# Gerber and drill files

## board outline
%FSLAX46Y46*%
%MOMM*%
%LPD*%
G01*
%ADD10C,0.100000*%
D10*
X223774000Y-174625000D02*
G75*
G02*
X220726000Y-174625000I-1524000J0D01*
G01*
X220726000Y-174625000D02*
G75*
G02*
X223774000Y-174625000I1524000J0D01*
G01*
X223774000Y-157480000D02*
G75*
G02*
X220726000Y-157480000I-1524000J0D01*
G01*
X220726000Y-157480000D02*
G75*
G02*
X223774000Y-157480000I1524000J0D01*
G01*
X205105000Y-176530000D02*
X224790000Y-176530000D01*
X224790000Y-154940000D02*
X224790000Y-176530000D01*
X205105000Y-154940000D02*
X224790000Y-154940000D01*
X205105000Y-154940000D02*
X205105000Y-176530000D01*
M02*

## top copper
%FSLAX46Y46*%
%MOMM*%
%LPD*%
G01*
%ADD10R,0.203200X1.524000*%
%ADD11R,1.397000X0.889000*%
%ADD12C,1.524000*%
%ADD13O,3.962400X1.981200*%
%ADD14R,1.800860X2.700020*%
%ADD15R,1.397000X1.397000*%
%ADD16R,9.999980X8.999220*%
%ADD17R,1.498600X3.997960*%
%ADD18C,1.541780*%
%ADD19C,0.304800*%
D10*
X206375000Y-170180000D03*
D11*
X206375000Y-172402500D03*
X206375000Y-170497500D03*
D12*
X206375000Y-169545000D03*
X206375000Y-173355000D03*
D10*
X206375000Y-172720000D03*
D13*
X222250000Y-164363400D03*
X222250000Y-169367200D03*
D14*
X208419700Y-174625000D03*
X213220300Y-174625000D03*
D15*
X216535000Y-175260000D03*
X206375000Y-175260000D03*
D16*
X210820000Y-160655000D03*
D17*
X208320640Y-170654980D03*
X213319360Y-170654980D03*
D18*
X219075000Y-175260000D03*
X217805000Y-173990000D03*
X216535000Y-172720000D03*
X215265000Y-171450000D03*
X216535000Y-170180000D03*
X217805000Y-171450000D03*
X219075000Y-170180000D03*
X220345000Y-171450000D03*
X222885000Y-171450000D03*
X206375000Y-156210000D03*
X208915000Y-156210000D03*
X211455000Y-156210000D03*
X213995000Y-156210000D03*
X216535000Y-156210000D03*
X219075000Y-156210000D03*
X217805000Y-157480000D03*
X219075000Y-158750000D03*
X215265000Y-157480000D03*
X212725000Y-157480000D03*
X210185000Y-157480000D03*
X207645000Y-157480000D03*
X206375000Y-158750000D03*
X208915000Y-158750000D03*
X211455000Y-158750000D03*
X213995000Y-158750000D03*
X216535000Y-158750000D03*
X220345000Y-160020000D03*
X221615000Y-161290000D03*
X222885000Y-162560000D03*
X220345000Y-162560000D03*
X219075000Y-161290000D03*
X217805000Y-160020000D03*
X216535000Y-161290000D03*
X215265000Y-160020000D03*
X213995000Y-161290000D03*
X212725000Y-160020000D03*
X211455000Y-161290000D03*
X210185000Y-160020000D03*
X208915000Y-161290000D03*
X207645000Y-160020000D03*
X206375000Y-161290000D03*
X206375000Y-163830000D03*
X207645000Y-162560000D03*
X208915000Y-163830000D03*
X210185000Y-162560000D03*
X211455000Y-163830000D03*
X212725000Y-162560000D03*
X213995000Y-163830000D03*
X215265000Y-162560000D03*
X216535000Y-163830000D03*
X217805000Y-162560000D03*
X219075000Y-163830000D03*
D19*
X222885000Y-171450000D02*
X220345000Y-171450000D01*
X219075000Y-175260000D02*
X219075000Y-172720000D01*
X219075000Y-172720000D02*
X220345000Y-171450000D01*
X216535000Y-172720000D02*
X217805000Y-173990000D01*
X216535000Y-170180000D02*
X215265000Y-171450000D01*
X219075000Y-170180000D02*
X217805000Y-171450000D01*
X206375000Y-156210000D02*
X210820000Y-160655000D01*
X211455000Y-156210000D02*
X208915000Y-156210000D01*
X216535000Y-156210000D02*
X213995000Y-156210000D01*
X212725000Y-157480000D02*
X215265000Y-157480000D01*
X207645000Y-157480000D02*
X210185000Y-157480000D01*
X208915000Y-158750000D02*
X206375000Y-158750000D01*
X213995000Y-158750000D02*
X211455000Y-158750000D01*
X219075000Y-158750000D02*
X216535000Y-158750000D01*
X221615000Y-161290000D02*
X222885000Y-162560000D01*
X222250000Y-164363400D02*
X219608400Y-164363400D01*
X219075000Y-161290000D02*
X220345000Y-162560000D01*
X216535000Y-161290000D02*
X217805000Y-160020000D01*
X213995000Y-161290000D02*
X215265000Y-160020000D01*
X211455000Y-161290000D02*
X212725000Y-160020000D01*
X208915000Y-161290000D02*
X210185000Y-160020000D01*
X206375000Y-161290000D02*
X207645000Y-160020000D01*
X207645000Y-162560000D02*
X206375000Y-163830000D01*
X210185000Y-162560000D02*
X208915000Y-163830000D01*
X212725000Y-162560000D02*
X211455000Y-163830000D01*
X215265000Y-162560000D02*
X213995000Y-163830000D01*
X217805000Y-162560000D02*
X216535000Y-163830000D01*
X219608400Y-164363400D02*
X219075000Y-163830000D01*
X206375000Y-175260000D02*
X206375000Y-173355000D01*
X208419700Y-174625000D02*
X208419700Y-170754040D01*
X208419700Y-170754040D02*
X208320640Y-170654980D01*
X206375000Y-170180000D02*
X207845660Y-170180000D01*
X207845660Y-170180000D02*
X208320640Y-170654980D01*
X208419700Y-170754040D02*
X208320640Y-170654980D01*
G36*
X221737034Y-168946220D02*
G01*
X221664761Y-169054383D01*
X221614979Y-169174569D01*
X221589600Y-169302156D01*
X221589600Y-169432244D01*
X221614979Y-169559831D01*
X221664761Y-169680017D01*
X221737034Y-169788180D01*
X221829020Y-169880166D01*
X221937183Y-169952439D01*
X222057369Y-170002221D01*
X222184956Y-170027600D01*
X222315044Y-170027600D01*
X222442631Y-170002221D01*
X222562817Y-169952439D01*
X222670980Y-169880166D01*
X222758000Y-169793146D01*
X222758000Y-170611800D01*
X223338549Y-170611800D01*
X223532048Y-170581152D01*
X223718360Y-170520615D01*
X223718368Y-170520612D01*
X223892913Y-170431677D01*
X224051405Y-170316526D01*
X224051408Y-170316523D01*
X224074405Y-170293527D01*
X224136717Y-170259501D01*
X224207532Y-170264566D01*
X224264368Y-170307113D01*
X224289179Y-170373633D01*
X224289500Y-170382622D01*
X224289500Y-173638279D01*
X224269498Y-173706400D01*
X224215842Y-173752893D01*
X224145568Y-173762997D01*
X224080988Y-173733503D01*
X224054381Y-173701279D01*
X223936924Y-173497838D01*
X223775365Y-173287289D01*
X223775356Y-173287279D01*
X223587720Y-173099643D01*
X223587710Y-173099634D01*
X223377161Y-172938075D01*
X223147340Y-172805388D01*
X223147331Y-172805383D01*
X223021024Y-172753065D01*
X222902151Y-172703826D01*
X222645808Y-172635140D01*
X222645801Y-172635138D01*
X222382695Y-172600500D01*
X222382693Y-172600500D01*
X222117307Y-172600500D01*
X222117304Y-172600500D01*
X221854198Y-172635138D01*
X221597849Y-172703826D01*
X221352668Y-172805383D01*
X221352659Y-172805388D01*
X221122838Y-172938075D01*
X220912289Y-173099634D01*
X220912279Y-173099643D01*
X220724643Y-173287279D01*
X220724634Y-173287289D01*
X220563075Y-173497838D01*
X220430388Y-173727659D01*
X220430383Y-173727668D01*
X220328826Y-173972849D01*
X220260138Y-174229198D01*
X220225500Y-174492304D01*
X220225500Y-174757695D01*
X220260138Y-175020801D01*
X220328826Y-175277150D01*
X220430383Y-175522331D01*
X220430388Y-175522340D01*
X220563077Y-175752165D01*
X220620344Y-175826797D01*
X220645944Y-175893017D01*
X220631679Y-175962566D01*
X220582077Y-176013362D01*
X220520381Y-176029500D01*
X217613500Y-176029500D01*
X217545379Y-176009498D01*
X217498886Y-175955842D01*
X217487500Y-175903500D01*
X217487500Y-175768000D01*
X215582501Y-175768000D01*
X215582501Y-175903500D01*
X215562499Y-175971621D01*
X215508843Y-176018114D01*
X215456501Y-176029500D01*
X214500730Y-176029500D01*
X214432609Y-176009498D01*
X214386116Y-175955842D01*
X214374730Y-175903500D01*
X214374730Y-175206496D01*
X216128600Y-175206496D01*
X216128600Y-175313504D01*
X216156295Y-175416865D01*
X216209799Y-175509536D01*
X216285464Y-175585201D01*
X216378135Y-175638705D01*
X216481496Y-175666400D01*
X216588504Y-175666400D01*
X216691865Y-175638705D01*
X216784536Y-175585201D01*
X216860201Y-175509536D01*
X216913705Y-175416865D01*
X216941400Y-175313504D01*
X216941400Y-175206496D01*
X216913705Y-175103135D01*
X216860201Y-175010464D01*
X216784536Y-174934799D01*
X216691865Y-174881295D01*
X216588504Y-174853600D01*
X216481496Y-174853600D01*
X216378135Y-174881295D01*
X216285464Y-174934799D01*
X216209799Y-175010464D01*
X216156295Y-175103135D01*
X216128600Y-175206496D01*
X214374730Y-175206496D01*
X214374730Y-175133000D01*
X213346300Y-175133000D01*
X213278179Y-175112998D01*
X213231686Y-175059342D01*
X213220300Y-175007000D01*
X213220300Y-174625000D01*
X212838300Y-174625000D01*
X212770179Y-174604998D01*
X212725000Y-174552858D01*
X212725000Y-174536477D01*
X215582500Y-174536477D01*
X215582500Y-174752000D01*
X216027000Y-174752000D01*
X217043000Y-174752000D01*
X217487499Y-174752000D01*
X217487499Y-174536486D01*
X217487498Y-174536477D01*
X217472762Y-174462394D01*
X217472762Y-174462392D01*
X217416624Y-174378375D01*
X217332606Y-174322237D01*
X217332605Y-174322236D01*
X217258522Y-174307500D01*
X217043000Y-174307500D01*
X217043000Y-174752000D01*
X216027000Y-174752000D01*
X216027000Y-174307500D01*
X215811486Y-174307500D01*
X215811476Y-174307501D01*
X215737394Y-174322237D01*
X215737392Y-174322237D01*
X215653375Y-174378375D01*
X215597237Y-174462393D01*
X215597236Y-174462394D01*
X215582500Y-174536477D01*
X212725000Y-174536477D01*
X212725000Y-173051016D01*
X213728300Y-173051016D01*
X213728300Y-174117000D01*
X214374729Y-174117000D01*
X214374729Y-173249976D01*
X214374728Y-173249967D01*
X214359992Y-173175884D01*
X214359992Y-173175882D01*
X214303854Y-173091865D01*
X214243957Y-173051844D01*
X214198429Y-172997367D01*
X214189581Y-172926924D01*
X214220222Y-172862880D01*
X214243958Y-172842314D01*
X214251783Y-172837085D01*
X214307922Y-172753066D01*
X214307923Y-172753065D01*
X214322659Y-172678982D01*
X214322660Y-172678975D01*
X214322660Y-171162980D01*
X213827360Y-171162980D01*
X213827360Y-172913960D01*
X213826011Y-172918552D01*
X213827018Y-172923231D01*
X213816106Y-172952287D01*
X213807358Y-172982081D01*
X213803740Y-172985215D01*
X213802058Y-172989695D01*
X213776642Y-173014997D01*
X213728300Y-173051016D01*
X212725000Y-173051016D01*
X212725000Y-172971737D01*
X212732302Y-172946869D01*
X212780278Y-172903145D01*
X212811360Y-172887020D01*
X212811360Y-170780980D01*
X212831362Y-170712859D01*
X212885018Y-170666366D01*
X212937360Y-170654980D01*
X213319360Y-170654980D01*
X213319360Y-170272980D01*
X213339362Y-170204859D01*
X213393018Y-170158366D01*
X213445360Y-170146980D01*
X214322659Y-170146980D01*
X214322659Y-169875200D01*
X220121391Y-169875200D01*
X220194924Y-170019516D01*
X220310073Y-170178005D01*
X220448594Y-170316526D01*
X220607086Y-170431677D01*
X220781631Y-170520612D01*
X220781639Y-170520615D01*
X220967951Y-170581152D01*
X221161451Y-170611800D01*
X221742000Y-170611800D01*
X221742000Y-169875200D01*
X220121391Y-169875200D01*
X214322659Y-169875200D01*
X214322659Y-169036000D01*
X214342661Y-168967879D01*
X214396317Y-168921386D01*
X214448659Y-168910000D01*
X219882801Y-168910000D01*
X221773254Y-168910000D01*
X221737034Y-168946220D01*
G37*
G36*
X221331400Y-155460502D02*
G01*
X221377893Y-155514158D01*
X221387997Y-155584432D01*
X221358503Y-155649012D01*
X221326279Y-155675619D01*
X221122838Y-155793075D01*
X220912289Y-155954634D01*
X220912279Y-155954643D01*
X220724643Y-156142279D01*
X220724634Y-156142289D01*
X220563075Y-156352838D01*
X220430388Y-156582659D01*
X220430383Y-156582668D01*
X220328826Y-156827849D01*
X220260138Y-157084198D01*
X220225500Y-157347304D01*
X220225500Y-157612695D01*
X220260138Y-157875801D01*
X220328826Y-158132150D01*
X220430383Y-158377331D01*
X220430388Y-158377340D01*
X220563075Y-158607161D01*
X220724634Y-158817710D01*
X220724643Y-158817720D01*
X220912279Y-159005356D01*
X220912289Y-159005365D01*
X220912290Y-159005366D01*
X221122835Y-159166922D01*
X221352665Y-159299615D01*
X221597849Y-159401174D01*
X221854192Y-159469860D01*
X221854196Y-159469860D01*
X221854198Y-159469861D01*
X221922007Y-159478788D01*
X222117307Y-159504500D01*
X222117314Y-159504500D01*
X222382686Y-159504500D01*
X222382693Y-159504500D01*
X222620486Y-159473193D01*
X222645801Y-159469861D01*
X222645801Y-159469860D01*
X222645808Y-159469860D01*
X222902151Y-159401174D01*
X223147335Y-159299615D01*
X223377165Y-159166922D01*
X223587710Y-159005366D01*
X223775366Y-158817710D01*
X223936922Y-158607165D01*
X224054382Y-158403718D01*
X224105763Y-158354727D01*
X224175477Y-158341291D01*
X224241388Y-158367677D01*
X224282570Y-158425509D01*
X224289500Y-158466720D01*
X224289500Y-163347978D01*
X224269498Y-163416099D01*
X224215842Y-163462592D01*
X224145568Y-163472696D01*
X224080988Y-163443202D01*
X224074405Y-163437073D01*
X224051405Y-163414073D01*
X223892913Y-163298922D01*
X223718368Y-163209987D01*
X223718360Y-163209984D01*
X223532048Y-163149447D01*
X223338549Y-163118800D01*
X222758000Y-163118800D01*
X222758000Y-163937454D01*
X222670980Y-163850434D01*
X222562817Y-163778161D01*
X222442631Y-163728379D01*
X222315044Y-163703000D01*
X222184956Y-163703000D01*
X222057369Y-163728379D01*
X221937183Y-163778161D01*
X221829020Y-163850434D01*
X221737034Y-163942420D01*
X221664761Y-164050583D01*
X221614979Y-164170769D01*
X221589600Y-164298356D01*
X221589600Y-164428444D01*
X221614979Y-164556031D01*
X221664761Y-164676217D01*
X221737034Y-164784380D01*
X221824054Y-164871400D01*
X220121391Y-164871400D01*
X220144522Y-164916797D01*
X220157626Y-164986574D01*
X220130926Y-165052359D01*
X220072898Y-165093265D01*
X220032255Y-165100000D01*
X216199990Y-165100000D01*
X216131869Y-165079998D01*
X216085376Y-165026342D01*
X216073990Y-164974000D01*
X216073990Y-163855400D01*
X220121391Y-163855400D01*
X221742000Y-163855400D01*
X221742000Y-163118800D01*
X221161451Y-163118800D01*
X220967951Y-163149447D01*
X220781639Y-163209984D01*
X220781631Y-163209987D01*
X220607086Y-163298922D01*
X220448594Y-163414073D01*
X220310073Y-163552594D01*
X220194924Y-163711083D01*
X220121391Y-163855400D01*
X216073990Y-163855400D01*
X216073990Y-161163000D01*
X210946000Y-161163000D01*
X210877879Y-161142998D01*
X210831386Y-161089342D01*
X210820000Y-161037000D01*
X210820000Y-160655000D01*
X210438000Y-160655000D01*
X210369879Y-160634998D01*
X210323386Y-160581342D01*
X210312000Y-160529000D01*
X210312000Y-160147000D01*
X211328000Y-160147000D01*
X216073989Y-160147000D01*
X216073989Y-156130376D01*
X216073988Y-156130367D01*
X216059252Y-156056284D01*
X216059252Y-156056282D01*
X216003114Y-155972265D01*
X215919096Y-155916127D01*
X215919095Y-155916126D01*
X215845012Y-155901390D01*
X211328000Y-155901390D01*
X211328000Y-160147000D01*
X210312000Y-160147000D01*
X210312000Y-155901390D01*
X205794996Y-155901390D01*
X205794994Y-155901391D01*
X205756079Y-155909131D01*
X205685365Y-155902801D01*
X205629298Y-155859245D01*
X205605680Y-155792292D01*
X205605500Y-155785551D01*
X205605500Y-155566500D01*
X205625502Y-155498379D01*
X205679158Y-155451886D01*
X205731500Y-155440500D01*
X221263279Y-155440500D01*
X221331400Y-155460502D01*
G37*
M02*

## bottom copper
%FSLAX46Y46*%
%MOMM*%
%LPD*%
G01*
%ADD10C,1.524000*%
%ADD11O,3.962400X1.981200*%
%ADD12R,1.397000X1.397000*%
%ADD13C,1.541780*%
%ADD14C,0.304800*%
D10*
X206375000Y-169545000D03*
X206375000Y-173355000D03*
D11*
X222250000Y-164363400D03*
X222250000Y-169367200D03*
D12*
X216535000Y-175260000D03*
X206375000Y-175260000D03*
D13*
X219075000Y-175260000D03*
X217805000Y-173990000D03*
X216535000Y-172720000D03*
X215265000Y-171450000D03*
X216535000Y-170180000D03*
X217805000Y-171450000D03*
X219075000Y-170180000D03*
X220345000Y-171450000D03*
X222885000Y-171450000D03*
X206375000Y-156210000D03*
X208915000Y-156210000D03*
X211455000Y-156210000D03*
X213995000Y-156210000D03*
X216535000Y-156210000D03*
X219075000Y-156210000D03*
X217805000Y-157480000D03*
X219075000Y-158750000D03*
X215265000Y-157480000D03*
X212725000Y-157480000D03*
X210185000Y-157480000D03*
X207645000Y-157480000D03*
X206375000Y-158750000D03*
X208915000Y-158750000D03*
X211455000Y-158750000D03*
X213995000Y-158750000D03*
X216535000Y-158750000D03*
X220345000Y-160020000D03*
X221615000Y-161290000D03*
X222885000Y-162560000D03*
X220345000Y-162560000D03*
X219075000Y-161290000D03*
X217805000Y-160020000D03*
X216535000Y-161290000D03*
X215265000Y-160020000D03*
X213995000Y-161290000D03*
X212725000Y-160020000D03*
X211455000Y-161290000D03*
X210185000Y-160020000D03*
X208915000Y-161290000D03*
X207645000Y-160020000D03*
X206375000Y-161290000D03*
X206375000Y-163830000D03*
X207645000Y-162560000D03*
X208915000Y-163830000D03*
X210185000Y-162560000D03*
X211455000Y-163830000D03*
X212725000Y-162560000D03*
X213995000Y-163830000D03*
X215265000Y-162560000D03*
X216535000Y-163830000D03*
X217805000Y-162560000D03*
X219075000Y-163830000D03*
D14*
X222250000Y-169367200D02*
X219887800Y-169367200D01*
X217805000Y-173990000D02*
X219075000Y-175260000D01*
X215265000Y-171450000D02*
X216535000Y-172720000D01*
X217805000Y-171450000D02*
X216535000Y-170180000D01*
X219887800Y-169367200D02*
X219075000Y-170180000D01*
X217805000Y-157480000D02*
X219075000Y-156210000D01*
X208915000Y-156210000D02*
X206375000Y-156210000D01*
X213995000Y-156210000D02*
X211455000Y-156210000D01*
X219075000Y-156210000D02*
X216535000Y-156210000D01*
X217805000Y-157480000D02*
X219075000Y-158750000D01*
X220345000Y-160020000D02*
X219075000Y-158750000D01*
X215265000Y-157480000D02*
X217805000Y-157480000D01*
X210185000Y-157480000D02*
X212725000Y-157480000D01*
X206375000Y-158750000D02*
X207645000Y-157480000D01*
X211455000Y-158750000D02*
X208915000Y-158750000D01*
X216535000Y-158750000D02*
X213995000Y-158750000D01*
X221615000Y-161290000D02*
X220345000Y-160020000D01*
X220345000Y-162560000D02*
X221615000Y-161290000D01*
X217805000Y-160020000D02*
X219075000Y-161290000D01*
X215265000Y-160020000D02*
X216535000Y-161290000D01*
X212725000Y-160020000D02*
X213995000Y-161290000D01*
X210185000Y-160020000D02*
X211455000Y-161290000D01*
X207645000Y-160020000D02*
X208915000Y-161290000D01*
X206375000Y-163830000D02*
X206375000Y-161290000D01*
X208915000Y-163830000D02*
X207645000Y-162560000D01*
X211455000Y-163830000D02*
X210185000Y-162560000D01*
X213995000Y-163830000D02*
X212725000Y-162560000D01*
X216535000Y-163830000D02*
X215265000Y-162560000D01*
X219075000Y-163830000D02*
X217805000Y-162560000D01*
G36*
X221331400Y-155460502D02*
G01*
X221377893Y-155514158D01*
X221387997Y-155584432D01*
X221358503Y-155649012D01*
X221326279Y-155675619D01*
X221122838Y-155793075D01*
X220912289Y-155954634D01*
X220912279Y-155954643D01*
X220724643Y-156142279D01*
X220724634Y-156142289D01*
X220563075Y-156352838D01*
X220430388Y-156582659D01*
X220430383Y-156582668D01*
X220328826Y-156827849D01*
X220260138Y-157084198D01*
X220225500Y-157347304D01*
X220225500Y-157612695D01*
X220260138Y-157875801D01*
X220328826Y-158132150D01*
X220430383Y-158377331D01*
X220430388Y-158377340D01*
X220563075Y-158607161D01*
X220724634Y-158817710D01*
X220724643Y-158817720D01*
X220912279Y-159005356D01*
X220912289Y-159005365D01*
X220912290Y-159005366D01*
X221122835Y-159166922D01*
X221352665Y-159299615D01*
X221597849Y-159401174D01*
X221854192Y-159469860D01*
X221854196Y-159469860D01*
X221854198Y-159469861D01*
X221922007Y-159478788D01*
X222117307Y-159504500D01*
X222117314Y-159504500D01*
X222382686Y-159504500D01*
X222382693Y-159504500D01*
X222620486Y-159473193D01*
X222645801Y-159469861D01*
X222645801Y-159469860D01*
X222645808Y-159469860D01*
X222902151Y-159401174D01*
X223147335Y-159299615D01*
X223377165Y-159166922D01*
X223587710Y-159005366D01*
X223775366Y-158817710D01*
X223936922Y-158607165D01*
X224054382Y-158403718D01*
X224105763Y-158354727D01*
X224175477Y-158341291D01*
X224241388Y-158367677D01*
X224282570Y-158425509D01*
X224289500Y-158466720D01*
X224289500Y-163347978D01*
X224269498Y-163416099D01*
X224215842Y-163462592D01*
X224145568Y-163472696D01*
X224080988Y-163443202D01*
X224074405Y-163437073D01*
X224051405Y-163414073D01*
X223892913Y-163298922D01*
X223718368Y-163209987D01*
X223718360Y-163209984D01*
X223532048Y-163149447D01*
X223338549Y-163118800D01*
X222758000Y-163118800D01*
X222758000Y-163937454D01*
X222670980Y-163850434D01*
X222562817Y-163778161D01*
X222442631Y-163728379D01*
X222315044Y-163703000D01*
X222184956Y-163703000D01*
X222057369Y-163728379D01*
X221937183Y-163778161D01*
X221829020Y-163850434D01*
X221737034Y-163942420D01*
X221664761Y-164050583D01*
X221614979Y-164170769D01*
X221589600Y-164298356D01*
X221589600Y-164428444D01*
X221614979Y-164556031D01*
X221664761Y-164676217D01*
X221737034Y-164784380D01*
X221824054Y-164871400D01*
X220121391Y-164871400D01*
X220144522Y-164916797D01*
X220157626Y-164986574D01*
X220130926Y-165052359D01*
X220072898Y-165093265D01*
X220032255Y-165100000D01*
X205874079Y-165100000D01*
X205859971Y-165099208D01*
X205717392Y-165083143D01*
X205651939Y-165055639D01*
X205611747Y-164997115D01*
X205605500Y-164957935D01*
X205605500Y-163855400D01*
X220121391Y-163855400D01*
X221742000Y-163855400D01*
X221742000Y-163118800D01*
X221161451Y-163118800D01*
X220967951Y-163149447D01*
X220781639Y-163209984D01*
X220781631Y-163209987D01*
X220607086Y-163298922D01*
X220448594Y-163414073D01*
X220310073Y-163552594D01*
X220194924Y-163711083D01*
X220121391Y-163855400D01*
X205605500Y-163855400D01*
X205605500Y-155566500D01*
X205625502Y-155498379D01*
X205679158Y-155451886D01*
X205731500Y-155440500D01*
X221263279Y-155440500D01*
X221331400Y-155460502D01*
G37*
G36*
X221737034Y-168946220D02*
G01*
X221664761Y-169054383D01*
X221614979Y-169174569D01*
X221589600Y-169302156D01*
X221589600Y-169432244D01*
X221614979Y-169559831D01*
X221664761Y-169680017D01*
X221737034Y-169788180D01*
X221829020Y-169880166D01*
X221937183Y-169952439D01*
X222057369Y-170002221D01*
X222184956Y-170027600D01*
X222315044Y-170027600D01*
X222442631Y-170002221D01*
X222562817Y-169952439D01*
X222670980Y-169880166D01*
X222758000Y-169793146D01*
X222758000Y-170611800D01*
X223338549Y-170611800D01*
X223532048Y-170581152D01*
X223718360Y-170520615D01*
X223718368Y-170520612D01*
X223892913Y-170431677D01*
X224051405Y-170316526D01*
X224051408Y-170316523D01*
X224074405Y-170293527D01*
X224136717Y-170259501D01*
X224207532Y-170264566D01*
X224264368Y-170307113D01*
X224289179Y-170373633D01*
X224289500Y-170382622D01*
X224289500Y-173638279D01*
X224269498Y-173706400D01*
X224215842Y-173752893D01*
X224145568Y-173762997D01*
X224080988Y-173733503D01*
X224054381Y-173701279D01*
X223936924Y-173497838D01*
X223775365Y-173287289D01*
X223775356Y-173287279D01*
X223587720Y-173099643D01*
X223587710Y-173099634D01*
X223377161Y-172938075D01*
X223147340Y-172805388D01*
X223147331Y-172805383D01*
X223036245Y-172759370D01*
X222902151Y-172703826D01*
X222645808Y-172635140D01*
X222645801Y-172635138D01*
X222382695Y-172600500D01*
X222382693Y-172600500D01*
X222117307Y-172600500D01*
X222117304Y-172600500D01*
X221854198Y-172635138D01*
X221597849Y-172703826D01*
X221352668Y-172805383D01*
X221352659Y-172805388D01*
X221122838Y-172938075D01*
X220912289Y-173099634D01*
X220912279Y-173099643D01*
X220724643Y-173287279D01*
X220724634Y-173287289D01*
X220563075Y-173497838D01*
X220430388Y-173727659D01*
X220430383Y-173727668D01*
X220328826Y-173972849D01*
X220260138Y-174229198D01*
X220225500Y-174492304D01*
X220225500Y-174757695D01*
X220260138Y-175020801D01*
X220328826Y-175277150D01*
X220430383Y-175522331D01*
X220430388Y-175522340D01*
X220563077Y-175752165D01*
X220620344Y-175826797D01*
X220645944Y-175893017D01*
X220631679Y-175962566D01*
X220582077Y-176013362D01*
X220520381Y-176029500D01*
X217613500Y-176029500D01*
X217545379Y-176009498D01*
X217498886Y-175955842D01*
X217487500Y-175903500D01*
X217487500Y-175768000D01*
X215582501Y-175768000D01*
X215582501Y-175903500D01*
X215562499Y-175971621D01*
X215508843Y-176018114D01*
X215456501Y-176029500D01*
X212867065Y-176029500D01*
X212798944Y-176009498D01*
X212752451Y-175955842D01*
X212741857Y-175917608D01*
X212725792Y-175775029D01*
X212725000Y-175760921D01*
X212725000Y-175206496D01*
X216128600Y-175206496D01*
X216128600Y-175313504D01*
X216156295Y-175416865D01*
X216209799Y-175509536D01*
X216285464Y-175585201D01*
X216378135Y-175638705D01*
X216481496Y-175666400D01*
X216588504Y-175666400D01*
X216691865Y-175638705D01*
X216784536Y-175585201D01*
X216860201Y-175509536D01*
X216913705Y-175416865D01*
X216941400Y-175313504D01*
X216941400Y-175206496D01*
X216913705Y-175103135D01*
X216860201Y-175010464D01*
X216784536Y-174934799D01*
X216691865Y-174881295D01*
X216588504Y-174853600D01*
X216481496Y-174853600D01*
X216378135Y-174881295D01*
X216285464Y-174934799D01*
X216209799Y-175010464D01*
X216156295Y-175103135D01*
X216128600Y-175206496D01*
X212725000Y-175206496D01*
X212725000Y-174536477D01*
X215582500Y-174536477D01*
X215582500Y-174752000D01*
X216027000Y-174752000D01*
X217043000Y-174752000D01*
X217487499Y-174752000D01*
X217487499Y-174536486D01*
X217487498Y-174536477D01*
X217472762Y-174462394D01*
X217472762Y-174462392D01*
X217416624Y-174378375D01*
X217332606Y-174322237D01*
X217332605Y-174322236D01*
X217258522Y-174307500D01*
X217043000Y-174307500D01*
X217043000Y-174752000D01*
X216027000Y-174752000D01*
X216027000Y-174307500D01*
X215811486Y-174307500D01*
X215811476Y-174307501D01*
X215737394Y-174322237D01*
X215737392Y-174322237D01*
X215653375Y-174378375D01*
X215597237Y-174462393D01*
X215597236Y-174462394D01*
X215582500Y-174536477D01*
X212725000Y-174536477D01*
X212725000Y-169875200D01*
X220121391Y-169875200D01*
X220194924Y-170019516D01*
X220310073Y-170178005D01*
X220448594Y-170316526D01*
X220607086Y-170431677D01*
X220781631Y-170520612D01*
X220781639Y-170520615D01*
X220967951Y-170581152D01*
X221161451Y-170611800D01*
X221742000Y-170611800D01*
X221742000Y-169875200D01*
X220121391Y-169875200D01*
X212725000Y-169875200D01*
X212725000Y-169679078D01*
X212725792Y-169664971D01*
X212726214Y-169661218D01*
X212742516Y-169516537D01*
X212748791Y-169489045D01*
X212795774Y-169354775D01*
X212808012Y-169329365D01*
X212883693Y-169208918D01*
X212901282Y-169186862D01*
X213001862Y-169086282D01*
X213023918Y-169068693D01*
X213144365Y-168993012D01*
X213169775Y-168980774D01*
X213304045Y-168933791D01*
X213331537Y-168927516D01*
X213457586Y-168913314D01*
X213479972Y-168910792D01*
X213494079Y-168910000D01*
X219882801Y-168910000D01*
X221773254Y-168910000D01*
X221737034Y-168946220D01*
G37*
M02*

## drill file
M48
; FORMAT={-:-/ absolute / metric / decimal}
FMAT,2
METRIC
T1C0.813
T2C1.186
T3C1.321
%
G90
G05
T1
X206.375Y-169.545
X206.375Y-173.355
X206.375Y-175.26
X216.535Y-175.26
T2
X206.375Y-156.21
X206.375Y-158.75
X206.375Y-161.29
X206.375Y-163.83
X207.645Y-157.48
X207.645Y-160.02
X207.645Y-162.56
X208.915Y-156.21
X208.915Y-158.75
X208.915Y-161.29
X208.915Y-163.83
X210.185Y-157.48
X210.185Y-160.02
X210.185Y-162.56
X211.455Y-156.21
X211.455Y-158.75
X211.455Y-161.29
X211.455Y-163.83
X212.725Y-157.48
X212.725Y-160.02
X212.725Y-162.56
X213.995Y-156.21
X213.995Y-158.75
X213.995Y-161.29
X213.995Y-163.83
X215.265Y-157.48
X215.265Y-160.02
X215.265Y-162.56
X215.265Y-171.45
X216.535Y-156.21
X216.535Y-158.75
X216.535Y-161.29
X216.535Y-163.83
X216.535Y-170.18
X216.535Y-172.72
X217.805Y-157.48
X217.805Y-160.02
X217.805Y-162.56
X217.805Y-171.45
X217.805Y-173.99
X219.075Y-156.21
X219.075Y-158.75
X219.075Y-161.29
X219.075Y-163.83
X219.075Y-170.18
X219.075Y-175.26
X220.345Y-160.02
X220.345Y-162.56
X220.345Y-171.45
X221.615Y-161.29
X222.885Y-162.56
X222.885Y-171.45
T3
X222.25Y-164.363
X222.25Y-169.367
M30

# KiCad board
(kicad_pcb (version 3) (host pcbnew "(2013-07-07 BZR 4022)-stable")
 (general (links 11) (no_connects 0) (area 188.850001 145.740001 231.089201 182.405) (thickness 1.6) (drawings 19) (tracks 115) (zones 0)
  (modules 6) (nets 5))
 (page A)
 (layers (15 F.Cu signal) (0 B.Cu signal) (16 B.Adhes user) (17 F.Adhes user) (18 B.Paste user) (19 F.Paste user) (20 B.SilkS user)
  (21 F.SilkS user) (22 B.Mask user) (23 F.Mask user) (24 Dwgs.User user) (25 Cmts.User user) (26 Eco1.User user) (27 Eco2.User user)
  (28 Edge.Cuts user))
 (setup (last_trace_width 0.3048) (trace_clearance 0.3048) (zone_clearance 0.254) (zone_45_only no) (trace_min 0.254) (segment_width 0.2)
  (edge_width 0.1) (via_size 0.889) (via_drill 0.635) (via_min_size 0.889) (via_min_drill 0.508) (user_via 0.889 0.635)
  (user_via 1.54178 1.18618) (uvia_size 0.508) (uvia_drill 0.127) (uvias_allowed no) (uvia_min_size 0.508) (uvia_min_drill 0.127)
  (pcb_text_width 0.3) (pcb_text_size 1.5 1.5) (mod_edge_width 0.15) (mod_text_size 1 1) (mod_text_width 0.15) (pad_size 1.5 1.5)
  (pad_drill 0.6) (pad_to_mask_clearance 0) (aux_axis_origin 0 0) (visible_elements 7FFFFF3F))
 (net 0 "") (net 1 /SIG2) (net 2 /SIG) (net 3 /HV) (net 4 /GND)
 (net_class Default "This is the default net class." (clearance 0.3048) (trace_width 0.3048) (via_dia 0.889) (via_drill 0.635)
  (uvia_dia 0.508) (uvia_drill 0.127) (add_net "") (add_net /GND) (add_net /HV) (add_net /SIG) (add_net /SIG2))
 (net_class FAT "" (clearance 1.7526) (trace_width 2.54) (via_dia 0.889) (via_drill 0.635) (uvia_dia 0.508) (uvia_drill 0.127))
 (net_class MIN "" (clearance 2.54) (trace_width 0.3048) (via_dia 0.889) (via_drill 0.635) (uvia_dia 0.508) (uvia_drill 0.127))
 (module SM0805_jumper (layer F.Cu) (at 206.375 171.45 90)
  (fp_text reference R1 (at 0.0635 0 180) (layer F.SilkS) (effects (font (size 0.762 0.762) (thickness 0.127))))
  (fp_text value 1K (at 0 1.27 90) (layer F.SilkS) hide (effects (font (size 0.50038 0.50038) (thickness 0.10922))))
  (pad 2 smd rect (at 1.27 0 90) (size 1.524 0.2032) (layers F.Cu F.Paste F.Mask) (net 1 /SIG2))
  (pad 1 smd rect (at -0.9525 0 90) (size 0.889 1.397) (layers F.Cu F.Paste F.Mask) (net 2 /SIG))
  (pad 2 smd rect (at 0.9525 0 90) (size 0.889 1.397) (layers F.Cu F.Paste F.Mask) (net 1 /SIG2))
  (pad 2 thru_hole circle (at 1.905 0 90) (size 1.524 1.524) (drill 0.8128) (layers *.Cu *.Mask F.SilkS) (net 1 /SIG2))
  (pad 1 thru_hole circle (at -1.905 0 90) (size 1.524 1.524) (drill 0.8128) (layers *.Cu *.Mask F.SilkS) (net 2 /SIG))
  (pad 1 smd rect (at -1.27 0 90) (size 1.524 0.2032) (layers F.Cu F.Paste F.Mask) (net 2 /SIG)))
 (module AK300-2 (layer F.Cu) (at 222.25 166.878 270)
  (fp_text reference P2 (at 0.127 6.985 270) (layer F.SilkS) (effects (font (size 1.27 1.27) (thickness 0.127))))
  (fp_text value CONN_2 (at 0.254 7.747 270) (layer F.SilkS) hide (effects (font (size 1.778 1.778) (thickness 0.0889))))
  (pad 1 thru_hole oval (at -2.5146 0 270) (size 1.9812 3.9624) (drill 1.3208) (layers *.Cu F.Paste F.SilkS F.Mask) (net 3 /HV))
  (pad 2 thru_hole oval (at 2.4892 0 270) (size 1.9812 3.9624) (drill 1.3208) (layers *.Cu F.Paste F.SilkS F.Mask) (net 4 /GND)))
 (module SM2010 (layer F.Cu) (at 210.82 174.625)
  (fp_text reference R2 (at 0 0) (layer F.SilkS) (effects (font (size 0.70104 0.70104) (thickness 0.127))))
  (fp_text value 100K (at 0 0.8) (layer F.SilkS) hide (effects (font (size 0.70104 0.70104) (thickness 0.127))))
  (pad 1 smd rect (at -2.4003 0) (size 1.80086 2.70002) (layers F.Cu F.Paste F.Mask) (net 1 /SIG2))
  (pad 2 smd rect (at 2.4003 0) (size 1.80086 2.70002) (layers F.Cu F.Paste F.Mask) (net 4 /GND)))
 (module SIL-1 (layer F.Cu) (at 216.535 175.26)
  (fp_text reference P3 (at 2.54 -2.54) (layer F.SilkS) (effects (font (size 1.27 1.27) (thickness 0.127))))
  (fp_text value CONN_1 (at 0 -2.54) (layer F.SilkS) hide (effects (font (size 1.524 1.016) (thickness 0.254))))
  (pad 1 thru_hole rect (at 0 0) (size 1.397 1.397) (drill 0.8128) (layers *.Cu *.Mask F.SilkS) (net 4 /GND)))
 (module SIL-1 (layer F.Cu) (at 206.375 175.26 180)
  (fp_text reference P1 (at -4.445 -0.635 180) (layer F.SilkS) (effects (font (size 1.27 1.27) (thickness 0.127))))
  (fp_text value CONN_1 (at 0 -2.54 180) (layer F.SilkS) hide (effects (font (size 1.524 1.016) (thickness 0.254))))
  (pad 1 thru_hole rect (at 0 0 180) (size 1.397 1.397) (drill 0.8128) (layers *.Cu *.Mask F.SilkS) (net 2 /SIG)))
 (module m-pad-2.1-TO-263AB (layer F.Cu) (at 210.82 160.655)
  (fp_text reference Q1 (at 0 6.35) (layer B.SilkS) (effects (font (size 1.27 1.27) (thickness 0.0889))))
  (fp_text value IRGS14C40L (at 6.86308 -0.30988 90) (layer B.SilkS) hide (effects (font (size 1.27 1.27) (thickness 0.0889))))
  (pad 2 smd rect (at 0 0) (size 9.99998 8.99922) (layers F.Cu F.Paste F.Mask) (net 3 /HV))
  (pad 1 smd rect (at -2.49936 9.99998) (size 1.4986 3.99796) (layers F.Cu F.Paste F.Mask) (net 1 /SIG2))
  (pad 3 smd rect (at 2.49936 9.99998) (size 1.4986 3.99796) (layers F.Cu F.Paste F.Mask) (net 4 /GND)))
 (gr_circle (center 222.25 174.625) (end 223.774 174.625) (layer Edge.Cuts) (width 0.1))
 (gr_circle (center 222.25 157.48) (end 223.774 157.48) (layer Edge.Cuts) (width 0.1))
 (gr_line (start 205.105 176.53) (end 224.79 176.53) (angle 90) (layer Edge.Cuts) (width 0.1))
 (gr_line (start 224.79 154.94) (end 224.79 176.53) (angle 90) (layer Edge.Cuts) (width 0.1))
 (gr_line (start 205.105 154.94) (end 224.79 154.94) (angle 90) (layer Edge.Cuts) (width 0.1))
 (gr_line (start 205.105 154.94) (end 205.105 176.53) (angle 90) (layer Edge.Cuts) (width 0.1))
 (segment (start 222.885 171.45) (end 220.345 171.45) (width 0.3048) (layer F.Cu) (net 4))
 (segment (start 219.075 175.26) (end 219.075 172.72) (width 0.3048) (layer F.Cu) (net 4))
 (segment (start 222.25 169.3672) (end 219.8878 169.3672) (width 0.3048) (layer B.Cu) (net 4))
 (segment (start 219.075 172.72) (end 220.345 171.45) (width 0.3048) (layer F.Cu) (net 4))
 (via (at 219.075 175.26) (size 1.54178) (drill 1.18618) (layers F.Cu B.Cu) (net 4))
 (segment (start 217.805 173.99) (end 219.075 175.26) (width 0.3048) (layer B.Cu) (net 4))
 (via (at 217.805 173.99) (size 1.54178) (drill 1.18618) (layers F.Cu B.Cu) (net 4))
 (segment (start 216.535 172.72) (end 217.805 173.99) (width 0.3048) (layer F.Cu) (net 4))
 (via (at 216.535 172.72) (size 1.54178) (drill 1.18618) (layers F.Cu B.Cu) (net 4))
 (segment (start 215.265 171.45) (end 216.535 172.72) (width 0.3048) (layer B.Cu) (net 4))
 (via (at 215.265 171.45) (size 1.54178) (drill 1.18618) (layers F.Cu B.Cu) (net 4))
 (segment (start 216.535 170.18) (end 215.265 171.45) (width 0.3048) (layer F.Cu) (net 4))
 (via (at 216.535 170.18) (size 1.54178) (drill 1.18618) (layers F.Cu B.Cu) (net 4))
 (segment (start 217.805 171.45) (end 216.535 170.18) (width 0.3048) (layer B.Cu) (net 4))
 (via (at 217.805 171.45) (size 1.54178) (drill 1.18618) (layers F.Cu B.Cu) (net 4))
 (segment (start 219.075 170.18) (end 217.805 171.45) (width 0.3048) (layer F.Cu) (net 4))
 (via (at 219.075 170.18) (size 1.54178) (drill 1.18618) (layers F.Cu B.Cu) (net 4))
 (segment (start 219.8878 169.3672) (end 219.075 170.18) (width 0.3048) (layer B.Cu) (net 4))
 (via (at 220.345 171.45) (size 1.54178) (drill 1.18618) (layers F.Cu B.Cu) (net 4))
 (via (at 222.885 171.45) (size 1.54178) (drill 1.18618) (layers F.Cu B.Cu) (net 4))
 (segment (start 217.805 157.48) (end 219.075 156.21) (width 0.3048) (layer B.Cu) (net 3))
 (segment (start 206.375 156.21) (end 210.82 160.655) (width 0.3048) (layer F.Cu) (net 3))
 (via (at 206.375 156.21) (size 1.54178) (drill 1.18618) (layers F.Cu B.Cu) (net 3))
 (segment (start 208.915 156.21) (end 206.375 156.21) (width 0.3048) (layer B.Cu) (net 3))
 (via (at 208.915 156.21) (size 1.54178) (drill 1.18618) (layers F.Cu B.Cu) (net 3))
 (segment (start 211.455 156.21) (end 208.915 156.21) (width 0.3048) (layer F.Cu) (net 3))
 (via (at 211.455 156.21) (size 1.54178) (drill 1.18618) (layers F.Cu B.Cu) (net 3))
 (segment (start 213.995 156.21) (end 211.455 156.21) (width 0.3048) (layer B.Cu) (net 3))
 (via (at 213.995 156.21) (size 1.54178) (drill 1.18618) (layers F.Cu B.Cu) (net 3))
 (segment (start 216.535 156.21) (end 213.995 156.21) (width 0.3048) (layer F.Cu) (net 3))
 (via (at 216.535 156.21) (size 1.54178) (drill 1.18618) (layers F.Cu B.Cu) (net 3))
 (segment (start 219.075 156.21) (end 216.535 156.21) (width 0.3048) (layer B.Cu) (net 3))
 (via (at 219.075 156.21) (size 1.54178) (drill 1.18618) (layers F.Cu B.Cu) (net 3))
 (via (at 217.805 157.48) (size 1.54178) (drill 1.18618) (layers F.Cu B.Cu) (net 3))
 (segment (start 217.805 157.48) (end 219.075 158.75) (width 0.3048) (layer B.Cu) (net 3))
 (segment (start 220.345 160.02) (end 219.075 158.75) (width 0.3048) (layer B.Cu) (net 3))
 (via (at 219.075 158.75) (size 1.54178) (drill 1.18618) (layers F.Cu B.Cu) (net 3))
 (segment (start 215.265 157.48) (end 217.805 157.48) (width 0.3048) (layer B.Cu) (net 3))
 (via (at 215.265 157.48) (size 1.54178) (drill 1.18618) (layers F.Cu B.Cu) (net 3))
 (segment (start 212.725 157.48) (end 215.265 157.48) (width 0.3048) (layer F.Cu) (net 3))
 (via (at 212.725 157.48) (size 1.54178) (drill 1.18618) (layers F.Cu B.Cu) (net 3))
 (segment (start 210.185 157.48) (end 212.725 157.48) (width 0.3048) (layer B.Cu) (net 3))
 (via (at 210.185 157.48) (size 1.54178) (drill 1.18618) (layers F.Cu B.Cu) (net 3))
 (segment (start 207.645 157.48) (end 210.185 157.48) (width 0.3048) (layer F.Cu) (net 3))
 (via (at 207.645 157.48) (size 1.54178) (drill 1.18618) (layers F.Cu B.Cu) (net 3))
 (segment (start 206.375 158.75) (end 207.645 157.48) (width 0.3048) (layer B.Cu) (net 3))
 (via (at 206.375 158.75) (size 1.54178) (drill 1.18618) (layers F.Cu B.Cu) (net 3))
 (segment (start 208.915 158.75) (end 206.375 158.75) (width 0.3048) (layer F.Cu) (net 3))
 (via (at 208.915 158.75) (size 1.54178) (drill 1.18618) (layers F.Cu B.Cu) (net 3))
 (segment (start 211.455 158.75) (end 208.915 158.75) (width 0.3048) (layer B.Cu) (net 3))
 (via (at 211.455 158.75) (size 1.54178) (drill 1.18618) (layers F.Cu B.Cu) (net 3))
 (segment (start 213.995 158.75) (end 211.455 158.75) (width 0.3048) (layer F.Cu) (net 3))
 (via (at 213.995 158.75) (size 1.54178) (drill 1.18618) (layers F.Cu B.Cu) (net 3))
 (segment (start 216.535 158.75) (end 213.995 158.75) (width 0.3048) (layer B.Cu) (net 3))
 (via (at 216.535 158.75) (size 1.54178) (drill 1.18618) (layers F.Cu B.Cu) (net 3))
 (segment (start 219.075 158.75) (end 216.535 158.75) (width 0.3048) (layer F.Cu) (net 3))
 (via (at 220.345 160.02) (size 1.54178) (drill 1.18618) (layers F.Cu B.Cu) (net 3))
 (segment (start 221.615 161.29) (end 220.345 160.02) (width 0.3048) (layer B.Cu) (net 3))
 (via (at 221.615 161.29) (size 1.54178) (drill 1.18618) (layers F.Cu B.Cu) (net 3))
 (via (at 222.885 162.56) (size 1.54178) (drill 1.18618) (layers F.Cu B.Cu) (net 3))
 (segment (start 221.615 161.29) (end 222.885 162.56) (width 0.3048) (layer F.Cu) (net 3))
 (segment (start 222.25 164.3634) (end 219.6084 164.3634) (width 0.3048) (layer F.Cu) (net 3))
 (segment (start 220.345 162.56) (end 221.615 161.29) (width 0.3048) (layer B.Cu) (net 3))
 (via (at 220.345 162.56) (size 1.54178) (drill 1.18618) (layers F.Cu B.Cu) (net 3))
 (segment (start 219.075 161.29) (end 220.345 162.56) (width 0.3048) (layer F.Cu) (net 3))
 (via (at 219.075 161.29) (size 1.54178) (drill 1.18618) (layers F.Cu B.Cu) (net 3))
 (segment (start 217.805 160.02) (end 219.075 161.29) (width 0.3048) (layer B.Cu) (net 3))
 (via (at 217.805 160.02) (size 1.54178) (drill 1.18618) (layers F.Cu B.Cu) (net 3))
 (segment (start 216.535 161.29) (end 217.805 160.02) (width 0.3048) (layer F.Cu) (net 3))
 (via (at 216.535 161.29) (size 1.54178) (drill 1.18618) (layers F.Cu B.Cu) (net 3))
 (segment (start 215.265 160.02) (end 216.535 161.29) (width 0.3048) (layer B.Cu) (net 3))
 (via (at 215.265 160.02) (size 1.54178) (drill 1.18618) (layers F.Cu B.Cu) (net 3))
 (segment (start 213.995 161.29) (end 215.265 160.02) (width 0.3048) (layer F.Cu) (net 3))
 (via (at 213.995 161.29) (size 1.54178) (drill 1.18618) (layers F.Cu B.Cu) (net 3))
 (segment (start 212.725 160.02) (end 213.995 161.29) (width 0.3048) (layer B.Cu) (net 3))
 (via (at 212.725 160.02) (size 1.54178) (drill 1.18618) (layers F.Cu B.Cu) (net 3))
 (segment (start 211.455 161.29) (end 212.725 160.02) (width 0.3048) (layer F.Cu) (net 3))
 (via (at 211.455 161.29) (size 1.54178) (drill 1.18618) (layers F.Cu B.Cu) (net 3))
 (segment (start 210.185 160.02) (end 211.455 161.29) (width 0.3048) (layer B.Cu) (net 3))
 (via (at 210.185 160.02) (size 1.54178) (drill 1.18618) (layers F.Cu B.Cu) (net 3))
 (segment (start 208.915 161.29) (end 210.185 160.02) (width 0.3048) (layer F.Cu) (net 3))
 (via (at 208.915 161.29) (size 1.54178) (drill 1.18618) (layers F.Cu B.Cu) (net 3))
 (segment (start 207.645 160.02) (end 208.915 161.29) (width 0.3048) (layer B.Cu) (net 3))
 (via (at 207.645 160.02) (size 1.54178) (drill 1.18618) (layers F.Cu B.Cu) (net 3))
 (segment (start 206.375 161.29) (end 207.645 160.02) (width 0.3048) (layer F.Cu) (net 3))
 (via (at 206.375 161.29) (size 1.54178) (drill 1.18618) (layers F.Cu B.Cu) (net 3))
 (segment (start 206.375 163.83) (end 206.375 161.29) (width 0.3048) (layer B.Cu) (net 3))
 (via (at 206.375 163.83) (size 1.54178) (drill 1.18618) (layers F.Cu B.Cu) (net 3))
 (segment (start 207.645 162.56) (end 206.375 163.83) (width 0.3048) (layer F.Cu) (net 3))
 (via (at 207.645 162.56) (size 1.54178) (drill 1.18618) (layers F.Cu B.Cu) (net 3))
 (segment (start 208.915 163.83) (end 207.645 162.56) (width 0.3048) (layer B.Cu) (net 3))
 (via (at 208.915 163.83) (size 1.54178) (drill 1.18618) (layers F.Cu B.Cu) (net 3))
 (segment (start 210.185 162.56) (end 208.915 163.83) (width 0.3048) (layer F.Cu) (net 3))
 (via (at 210.185 162.56) (size 1.54178) (drill 1.18618) (layers F.Cu B.Cu) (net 3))
 (segment (start 211.455 163.83) (end 210.185 162.56) (width 0.3048) (layer B.Cu) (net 3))
 (via (at 211.455 163.83) (size 1.54178) (drill 1.18618) (layers F.Cu B.Cu) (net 3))
 (segment (start 212.725 162.56) (end 211.455 163.83) (width 0.3048) (layer F.Cu) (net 3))
 (via (at 212.725 162.56) (size 1.54178) (drill 1.18618) (layers F.Cu B.Cu) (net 3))
 (segment (start 213.995 163.83) (end 212.725 162.56) (width 0.3048) (layer B.Cu) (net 3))
 (via (at 213.995 163.83) (size 1.54178) (drill 1.18618) (layers F.Cu B.Cu) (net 3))
 (segment (start 215.265 162.56) (end 213.995 163.83) (width 0.3048) (layer F.Cu) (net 3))
 (via (at 215.265 162.56) (size 1.54178) (drill 1.18618) (layers F.Cu B.Cu) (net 3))
 (segment (start 216.535 163.83) (end 215.265 162.56) (width 0.3048) (layer B.Cu) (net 3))
 (via (at 216.535 163.83) (size 1.54178) (drill 1.18618) (layers F.Cu B.Cu) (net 3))
 (segment (start 217.805 162.56) (end 216.535 163.83) (width 0.3048) (layer F.Cu) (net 3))
 (via (at 217.805 162.56) (size 1.54178) (drill 1.18618) (layers F.Cu B.Cu) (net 3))
 (segment (start 219.075 163.83) (end 217.805 162.56) (width 0.3048) (layer B.Cu) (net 3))
 (via (at 219.075 163.83) (size 1.54178) (drill 1.18618) (layers F.Cu B.Cu) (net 3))
 (segment (start 219.6084 164.3634) (end 219.075 163.83) (width 0.3048) (layer F.Cu) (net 3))
 (segment (start 206.375 175.26) (end 206.375 173.355) (width 0.3048) (layer F.Cu) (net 2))
 (segment (start 208.4197 174.625) (end 208.4197 170.75404) (width 0.3048) (layer F.Cu) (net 1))
 (segment (start 208.4197 170.75404) (end 208.32064 170.65498) (width 0.3048) (layer F.Cu) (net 1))
 (segment (start 206.375 170.18) (end 207.84566 170.18) (width 0.3048) (layer F.Cu) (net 1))
 (segment (start 207.84566 170.18) (end 208.32064 170.65498) (width 0.3048) (layer F.Cu) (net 1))
 (segment (start 208.4197 170.75404) (end 208.32064 170.65498) (width 0.3048) (layer F.Cu) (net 1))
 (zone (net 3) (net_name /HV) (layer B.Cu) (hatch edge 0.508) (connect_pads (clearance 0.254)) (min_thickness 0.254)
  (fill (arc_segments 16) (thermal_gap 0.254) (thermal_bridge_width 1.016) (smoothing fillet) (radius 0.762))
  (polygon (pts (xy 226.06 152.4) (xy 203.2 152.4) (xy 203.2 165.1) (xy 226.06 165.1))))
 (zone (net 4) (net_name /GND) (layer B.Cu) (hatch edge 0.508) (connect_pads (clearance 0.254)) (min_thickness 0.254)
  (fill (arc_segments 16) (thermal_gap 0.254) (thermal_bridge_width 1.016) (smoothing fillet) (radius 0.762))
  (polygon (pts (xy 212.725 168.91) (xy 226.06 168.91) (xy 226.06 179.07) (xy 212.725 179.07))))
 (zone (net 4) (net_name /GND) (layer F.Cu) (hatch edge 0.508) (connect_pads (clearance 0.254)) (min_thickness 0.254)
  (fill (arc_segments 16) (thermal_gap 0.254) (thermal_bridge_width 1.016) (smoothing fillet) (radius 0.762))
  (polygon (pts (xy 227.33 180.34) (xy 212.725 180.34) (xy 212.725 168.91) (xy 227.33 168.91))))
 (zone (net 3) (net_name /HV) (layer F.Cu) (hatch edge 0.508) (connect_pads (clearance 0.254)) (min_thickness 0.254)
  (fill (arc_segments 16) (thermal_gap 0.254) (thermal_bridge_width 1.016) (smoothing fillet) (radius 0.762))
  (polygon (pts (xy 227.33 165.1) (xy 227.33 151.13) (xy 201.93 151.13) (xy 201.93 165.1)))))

